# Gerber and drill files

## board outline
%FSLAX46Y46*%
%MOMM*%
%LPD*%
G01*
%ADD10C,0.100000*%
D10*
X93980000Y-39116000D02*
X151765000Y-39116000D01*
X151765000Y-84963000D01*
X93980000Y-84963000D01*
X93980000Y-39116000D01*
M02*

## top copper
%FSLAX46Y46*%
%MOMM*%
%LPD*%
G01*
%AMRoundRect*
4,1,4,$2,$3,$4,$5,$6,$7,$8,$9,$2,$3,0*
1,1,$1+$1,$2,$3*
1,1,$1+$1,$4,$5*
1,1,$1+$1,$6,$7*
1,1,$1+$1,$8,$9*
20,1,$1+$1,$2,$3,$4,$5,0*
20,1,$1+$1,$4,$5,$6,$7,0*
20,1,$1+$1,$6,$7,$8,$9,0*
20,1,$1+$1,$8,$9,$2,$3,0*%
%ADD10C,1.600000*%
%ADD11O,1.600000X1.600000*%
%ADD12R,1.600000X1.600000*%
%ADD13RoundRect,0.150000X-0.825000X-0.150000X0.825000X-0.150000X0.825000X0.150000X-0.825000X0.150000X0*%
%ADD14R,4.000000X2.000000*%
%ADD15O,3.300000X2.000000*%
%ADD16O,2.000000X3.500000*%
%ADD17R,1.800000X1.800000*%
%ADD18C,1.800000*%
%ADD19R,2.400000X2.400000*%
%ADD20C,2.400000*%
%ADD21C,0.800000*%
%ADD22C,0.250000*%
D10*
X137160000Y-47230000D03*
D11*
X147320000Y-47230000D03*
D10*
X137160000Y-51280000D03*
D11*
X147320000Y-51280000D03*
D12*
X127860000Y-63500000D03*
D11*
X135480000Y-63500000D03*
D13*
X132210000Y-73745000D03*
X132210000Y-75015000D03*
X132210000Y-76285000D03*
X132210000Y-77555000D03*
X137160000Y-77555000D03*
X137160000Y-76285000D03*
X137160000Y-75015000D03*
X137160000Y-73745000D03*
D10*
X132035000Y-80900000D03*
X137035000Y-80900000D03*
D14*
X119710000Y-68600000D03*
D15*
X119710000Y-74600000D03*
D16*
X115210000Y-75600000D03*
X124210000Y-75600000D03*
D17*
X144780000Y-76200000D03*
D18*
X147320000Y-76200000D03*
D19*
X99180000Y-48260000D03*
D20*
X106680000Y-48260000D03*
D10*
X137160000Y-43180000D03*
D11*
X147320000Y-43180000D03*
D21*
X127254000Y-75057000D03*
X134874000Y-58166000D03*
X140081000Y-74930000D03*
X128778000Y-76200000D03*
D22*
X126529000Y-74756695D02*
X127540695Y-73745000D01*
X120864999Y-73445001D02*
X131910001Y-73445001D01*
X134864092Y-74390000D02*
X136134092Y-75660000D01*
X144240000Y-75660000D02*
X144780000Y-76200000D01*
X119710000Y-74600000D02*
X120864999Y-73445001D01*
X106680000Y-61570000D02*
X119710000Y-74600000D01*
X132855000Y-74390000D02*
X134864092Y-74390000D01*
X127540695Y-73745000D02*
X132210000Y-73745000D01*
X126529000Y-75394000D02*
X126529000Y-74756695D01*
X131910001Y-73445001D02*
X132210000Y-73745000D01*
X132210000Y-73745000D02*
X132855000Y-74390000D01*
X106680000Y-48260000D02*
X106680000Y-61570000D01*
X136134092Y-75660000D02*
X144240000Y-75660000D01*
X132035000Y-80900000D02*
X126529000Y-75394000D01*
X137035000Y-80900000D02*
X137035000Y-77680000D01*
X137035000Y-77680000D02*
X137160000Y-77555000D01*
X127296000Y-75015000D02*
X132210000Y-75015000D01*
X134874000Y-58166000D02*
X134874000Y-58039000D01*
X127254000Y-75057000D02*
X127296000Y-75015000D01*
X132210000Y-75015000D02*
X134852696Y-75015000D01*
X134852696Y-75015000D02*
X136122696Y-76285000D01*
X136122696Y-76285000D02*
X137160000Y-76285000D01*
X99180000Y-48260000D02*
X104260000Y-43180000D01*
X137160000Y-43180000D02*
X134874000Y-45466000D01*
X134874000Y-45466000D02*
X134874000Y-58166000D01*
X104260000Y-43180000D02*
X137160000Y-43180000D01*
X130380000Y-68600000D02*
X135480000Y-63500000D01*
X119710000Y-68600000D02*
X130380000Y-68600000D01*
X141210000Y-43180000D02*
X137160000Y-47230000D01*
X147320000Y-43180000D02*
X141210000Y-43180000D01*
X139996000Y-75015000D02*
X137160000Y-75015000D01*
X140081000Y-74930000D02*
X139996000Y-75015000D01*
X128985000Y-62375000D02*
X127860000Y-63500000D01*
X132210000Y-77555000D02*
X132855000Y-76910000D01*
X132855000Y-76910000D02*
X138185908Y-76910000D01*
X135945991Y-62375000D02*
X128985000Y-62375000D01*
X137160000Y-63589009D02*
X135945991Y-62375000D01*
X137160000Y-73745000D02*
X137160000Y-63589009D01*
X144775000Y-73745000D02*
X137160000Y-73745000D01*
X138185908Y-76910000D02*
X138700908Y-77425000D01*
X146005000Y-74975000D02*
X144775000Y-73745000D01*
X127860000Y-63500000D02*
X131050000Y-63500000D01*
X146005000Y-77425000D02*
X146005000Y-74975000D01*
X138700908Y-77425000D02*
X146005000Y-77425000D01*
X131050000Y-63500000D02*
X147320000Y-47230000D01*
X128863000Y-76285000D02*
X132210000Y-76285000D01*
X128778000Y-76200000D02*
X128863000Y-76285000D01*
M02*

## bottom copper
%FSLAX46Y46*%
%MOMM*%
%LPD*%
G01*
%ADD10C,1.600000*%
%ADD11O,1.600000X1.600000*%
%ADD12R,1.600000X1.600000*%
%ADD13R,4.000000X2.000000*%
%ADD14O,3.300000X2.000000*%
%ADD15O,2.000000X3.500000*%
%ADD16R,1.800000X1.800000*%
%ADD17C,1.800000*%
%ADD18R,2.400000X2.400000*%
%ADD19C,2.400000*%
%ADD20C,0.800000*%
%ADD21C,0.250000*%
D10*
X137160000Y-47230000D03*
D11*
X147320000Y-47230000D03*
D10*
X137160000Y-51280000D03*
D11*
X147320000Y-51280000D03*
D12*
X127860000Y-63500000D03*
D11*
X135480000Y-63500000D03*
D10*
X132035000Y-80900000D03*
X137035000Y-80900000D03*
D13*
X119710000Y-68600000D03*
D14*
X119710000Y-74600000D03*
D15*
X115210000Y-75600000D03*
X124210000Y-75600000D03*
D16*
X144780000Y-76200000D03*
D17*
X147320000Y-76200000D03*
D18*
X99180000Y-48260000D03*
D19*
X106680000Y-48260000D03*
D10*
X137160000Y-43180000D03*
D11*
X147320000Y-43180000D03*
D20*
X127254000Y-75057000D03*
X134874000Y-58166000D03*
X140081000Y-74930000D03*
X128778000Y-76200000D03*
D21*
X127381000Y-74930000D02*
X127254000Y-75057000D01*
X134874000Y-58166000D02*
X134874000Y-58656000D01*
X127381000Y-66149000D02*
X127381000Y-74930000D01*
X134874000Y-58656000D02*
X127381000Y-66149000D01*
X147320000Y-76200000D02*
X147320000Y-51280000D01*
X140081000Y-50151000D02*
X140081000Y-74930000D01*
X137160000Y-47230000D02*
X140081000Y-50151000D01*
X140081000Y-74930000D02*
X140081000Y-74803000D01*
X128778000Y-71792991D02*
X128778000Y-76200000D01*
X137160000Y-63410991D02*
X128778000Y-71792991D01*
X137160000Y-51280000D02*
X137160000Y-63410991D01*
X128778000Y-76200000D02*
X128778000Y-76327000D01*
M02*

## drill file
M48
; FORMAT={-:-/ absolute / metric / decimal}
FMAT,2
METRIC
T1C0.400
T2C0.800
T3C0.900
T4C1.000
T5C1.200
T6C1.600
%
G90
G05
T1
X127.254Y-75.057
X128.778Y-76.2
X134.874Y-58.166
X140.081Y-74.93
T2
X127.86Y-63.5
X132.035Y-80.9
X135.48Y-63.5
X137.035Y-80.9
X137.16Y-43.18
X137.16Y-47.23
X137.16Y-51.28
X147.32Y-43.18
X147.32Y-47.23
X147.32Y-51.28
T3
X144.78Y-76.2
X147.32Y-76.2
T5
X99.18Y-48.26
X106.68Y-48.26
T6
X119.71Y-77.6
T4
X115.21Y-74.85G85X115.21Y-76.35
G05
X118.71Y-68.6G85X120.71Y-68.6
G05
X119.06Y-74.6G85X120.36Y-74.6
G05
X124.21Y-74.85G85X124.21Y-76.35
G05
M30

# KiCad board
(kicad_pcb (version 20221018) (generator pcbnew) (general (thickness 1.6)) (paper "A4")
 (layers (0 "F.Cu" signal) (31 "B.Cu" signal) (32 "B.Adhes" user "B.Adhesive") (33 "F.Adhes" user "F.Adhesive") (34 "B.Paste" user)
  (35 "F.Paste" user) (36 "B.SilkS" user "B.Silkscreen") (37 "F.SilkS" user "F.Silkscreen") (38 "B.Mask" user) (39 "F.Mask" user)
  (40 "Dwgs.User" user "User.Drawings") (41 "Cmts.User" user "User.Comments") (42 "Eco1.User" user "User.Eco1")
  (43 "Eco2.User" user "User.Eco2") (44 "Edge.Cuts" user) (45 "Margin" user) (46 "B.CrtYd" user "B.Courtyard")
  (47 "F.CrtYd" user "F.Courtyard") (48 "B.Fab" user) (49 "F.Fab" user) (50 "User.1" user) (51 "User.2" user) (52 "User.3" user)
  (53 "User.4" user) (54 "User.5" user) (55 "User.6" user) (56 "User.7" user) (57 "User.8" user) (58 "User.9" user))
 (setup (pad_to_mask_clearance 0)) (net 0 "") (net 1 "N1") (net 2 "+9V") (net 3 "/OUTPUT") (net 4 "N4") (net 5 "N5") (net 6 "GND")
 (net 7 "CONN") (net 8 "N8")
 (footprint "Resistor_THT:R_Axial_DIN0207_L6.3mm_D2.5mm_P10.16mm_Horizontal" (layer "F.Cu") (at 137.16 47.23)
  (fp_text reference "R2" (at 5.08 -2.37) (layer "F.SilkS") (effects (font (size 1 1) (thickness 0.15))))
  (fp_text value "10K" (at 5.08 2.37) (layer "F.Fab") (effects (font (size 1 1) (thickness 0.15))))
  (pad "1" thru_hole circle (at 0 0) (size 1.6 1.6) (drill 0.8) (layers "*.Cu" "*.Mask") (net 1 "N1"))
  (pad "2" thru_hole oval (at 10.16 0) (size 1.6 1.6) (drill 0.8) (layers "*.Cu" "*.Mask") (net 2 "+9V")))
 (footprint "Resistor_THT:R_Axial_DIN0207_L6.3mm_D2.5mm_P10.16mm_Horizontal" (layer "F.Cu") (at 137.16 51.28)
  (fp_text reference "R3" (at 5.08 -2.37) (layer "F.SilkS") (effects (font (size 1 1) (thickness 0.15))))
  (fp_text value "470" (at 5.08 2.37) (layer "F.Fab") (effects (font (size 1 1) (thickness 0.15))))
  (pad "1" thru_hole circle (at 0 0) (size 1.6 1.6) (drill 0.8) (layers "*.Cu" "*.Mask") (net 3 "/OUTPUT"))
  (pad "2" thru_hole oval (at 10.16 0) (size 1.6 1.6) (drill 0.8) (layers "*.Cu" "*.Mask") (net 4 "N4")))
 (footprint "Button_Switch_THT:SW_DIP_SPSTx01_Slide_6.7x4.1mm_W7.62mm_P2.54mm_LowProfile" (layer "F.Cu") (at 127.86 63.5)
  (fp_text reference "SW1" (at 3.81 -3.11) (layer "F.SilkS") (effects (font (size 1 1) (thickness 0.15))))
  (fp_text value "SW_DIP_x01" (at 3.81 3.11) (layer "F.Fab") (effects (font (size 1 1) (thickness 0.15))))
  (pad "1" thru_hole rect (at 0 0) (size 1.6 1.6) (drill 0.8) (layers "*.Cu" "*.Mask") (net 2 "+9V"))
  (pad "2" thru_hole oval (at 7.62 0) (size 1.6 1.6) (drill 0.8) (layers "*.Cu" "*.Mask") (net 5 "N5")))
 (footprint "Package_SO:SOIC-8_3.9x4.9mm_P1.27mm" (layer "F.Cu") (at 134.685 75.65)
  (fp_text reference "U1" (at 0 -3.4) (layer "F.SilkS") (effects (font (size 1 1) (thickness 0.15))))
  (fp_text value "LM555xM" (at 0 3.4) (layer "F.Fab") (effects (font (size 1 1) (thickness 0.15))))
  (pad "1" smd roundrect (at -2.475 -1.905) (size 1.95 0.6) (layers "F.Cu" "F.Paste" "F.Mask") (roundrect_rratio 0.25) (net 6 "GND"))
  (pad "2" smd roundrect (at -2.475 -0.635) (size 1.95 0.6) (layers "F.Cu" "F.Paste" "F.Mask") (roundrect_rratio 0.25) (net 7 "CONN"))
  (pad "3" smd roundrect (at -2.475 0.635) (size 1.95 0.6) (layers "F.Cu" "F.Paste" "F.Mask") (roundrect_rratio 0.25) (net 3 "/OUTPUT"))
  (pad "4" smd roundrect (at -2.475 1.905) (size 1.95 0.6) (layers "F.Cu" "F.Paste" "F.Mask") (roundrect_rratio 0.25) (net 2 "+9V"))
  (pad "5" smd roundrect (at 2.475 1.905) (size 1.95 0.6) (layers "F.Cu" "F.Paste" "F.Mask") (roundrect_rratio 0.25) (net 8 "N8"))
  (pad "6" smd roundrect (at 2.475 0.635) (size 1.95 0.6) (layers "F.Cu" "F.Paste" "F.Mask") (roundrect_rratio 0.25) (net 7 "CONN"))
  (pad "7" smd roundrect (at 2.475 -0.635) (size 1.95 0.6) (layers "F.Cu" "F.Paste" "F.Mask") (roundrect_rratio 0.25) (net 1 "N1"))
  (pad "8" smd roundrect (at 2.475 -1.905) (size 1.95 0.6) (layers "F.Cu" "F.Paste" "F.Mask") (roundrect_rratio 0.25) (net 2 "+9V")))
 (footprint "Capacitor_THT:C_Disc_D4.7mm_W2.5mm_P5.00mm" (layer "F.Cu") (at 132.035 80.9)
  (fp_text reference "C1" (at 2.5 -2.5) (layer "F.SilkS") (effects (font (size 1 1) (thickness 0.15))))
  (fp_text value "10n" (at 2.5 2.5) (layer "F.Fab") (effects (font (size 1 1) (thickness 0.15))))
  (pad "1" thru_hole circle (at 0 0) (size 1.6 1.6) (drill 0.8) (layers "*.Cu" "*.Mask") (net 6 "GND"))
  (pad "2" thru_hole circle (at 5 0) (size 1.6 1.6) (drill 0.8) (layers "*.Cu" "*.Mask") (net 8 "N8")))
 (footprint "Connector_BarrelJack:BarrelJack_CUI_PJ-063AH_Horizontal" (layer "F.Cu") (at 119.71 68.6)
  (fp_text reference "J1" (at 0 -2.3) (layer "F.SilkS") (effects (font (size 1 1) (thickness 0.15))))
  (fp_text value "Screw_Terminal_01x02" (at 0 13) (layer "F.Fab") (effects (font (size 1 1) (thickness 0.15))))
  (pad "" np_thru_hole circle (at 0 9) (size 1.6 1.6) (drill 1.6) (layers "*.Cu" "*.Mask"))
  (pad "1" thru_hole rect (at 0 0) (size 4 2) (drill oval 3 1) (layers "*.Cu" "*.Mask") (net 5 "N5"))
  (pad "2" thru_hole oval (at 0 6) (size 3.3 2) (drill oval 2.3 1) (layers "*.Cu" "*.Mask") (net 6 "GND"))
  (pad "MP" thru_hole oval (at -4.5 7) (size 2 3.5) (drill oval 1 2.5) (layers "*.Cu" "*.Mask"))
  (pad "MP" thru_hole oval (at 4.5 7) (size 2 3.5) (drill oval 1 2.5) (layers "*.Cu" "*.Mask")))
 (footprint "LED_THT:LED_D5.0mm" (layer "F.Cu") (at 144.78 76.2)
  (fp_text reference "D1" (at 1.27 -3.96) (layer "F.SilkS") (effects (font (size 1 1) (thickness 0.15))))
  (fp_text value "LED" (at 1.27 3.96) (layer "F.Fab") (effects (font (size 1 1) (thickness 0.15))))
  (pad "1" thru_hole rect (at 0 0) (size 1.8 1.8) (drill 0.9) (layers "*.Cu" "*.Mask") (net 6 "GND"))
  (pad "2" thru_hole circle (at 2.54 0) (size 1.8 1.8) (drill 0.9) (layers "*.Cu" "*.Mask") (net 4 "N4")))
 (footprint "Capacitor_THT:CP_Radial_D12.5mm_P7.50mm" (layer "F.Cu") (at 99.18 48.26)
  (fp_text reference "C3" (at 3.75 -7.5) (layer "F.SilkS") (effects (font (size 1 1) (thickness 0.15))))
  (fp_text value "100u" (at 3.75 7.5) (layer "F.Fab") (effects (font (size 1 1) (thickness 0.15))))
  (pad "1" thru_hole rect (at 0 0) (size 2.4 2.4) (drill 1.2) (layers "*.Cu" "*.Mask") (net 7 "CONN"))
  (pad "2" thru_hole circle (at 7.5 0) (size 2.4 2.4) (drill 1.2) (layers "*.Cu" "*.Mask") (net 6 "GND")))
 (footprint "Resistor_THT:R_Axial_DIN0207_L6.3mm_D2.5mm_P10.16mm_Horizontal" (layer "F.Cu") (at 137.16 43.18)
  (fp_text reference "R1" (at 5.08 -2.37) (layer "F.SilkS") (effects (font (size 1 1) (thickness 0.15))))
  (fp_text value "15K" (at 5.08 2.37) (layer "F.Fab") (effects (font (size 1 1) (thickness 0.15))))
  (pad "1" thru_hole circle (at 0 0) (size 1.6 1.6) (drill 0.8) (layers "*.Cu" "*.Mask") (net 7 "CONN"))
  (pad "2" thru_hole oval (at 10.16 0) (size 1.6 1.6) (drill 0.8) (layers "*.Cu" "*.Mask") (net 1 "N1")))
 (gr_rect (start 93.98 39.116) (end 151.765 84.963) (stroke (width 0.1) (type default)) (fill none) (layer "Edge.Cuts"))
 (segment (start 126.529 74.756695) (end 127.540695 73.745) (width 0.25) (layer "F.Cu") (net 6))
 (segment (start 120.864999 73.445001) (end 131.910001 73.445001) (width 0.25) (layer "F.Cu") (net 6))
 (segment (start 134.864092 74.39) (end 136.134092 75.66) (width 0.25) (layer "F.Cu") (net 6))
 (segment (start 144.24 75.66) (end 144.78 76.2) (width 0.25) (layer "F.Cu") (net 6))
 (segment (start 119.71 74.6) (end 120.864999 73.445001) (width 0.25) (layer "F.Cu") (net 6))
 (segment (start 106.68 61.57) (end 119.71 74.6) (width 0.25) (layer "F.Cu") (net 6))
 (segment (start 132.855 74.39) (end 134.864092 74.39) (width 0.25) (layer "F.Cu") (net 6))
 (segment (start 127.540695 73.745) (end 132.21 73.745) (width 0.25) (layer "F.Cu") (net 6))
 (segment (start 126.529 75.394) (end 126.529 74.756695) (width 0.25) (layer "F.Cu") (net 6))
 (segment (start 131.910001 73.445001) (end 132.21 73.745) (width 0.25) (layer "F.Cu") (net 6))
 (segment (start 132.21 73.745) (end 132.855 74.39) (width 0.25) (layer "F.Cu") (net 6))
 (segment (start 106.68 48.26) (end 106.68 61.57) (width 0.25) (layer "F.Cu") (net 6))
 (segment (start 136.134092 75.66) (end 144.24 75.66) (width 0.25) (layer "F.Cu") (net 6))
 (segment (start 132.035 80.9) (end 126.529 75.394) (width 0.25) (layer "F.Cu") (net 6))
 (segment (start 137.035 80.9) (end 137.035 77.68) (width 0.25) (layer "F.Cu") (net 8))
 (segment (start 137.035 77.68) (end 137.16 77.555) (width 0.25) (layer "F.Cu") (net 8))
 (segment (start 127.296 75.015) (end 132.21 75.015) (width 0.25) (layer "F.Cu") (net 7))
 (segment (start 134.874 58.166) (end 134.874 58.039) (width 0.25) (layer "F.Cu") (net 7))
 (segment (start 127.254 75.057) (end 127.296 75.015) (width 0.25) (layer "F.Cu") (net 7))
 (segment (start 132.21 75.015) (end 134.852696 75.015) (width 0.25) (layer "F.Cu") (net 7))
 (segment (start 134.852696 75.015) (end 136.122696 76.285) (width 0.25) (layer "F.Cu") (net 7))
 (segment (start 136.122696 76.285) (end 137.16 76.285) (width 0.25) (layer "F.Cu") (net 7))
 (segment (start 99.18 48.26) (end 104.26 43.18) (width 0.25) (layer "F.Cu") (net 7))
 (segment (start 137.16 43.18) (end 134.874 45.466) (width 0.25) (layer "F.Cu") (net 7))
 (segment (start 134.874 45.466) (end 134.874 58.166) (width 0.25) (layer "F.Cu") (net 7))
 (segment (start 104.26 43.18) (end 137.16 43.18) (width 0.25) (layer "F.Cu") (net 7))
 (via (at 127.254 75.057) (size 0.8) (drill 0.4) (layers "F.Cu" "B.Cu") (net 7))
 (via (at 134.874 58.166) (size 0.8) (drill 0.4) (layers "F.Cu" "B.Cu") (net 7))
 (segment (start 127.381 74.93) (end 127.254 75.057) (width 0.25) (layer "B.Cu") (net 7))
 (segment (start 134.874 58.166) (end 134.874 58.656) (width 0.25) (layer "B.Cu") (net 7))
 (segment (start 127.381 66.149) (end 127.381 74.93) (width 0.25) (layer "B.Cu") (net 7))
 (segment (start 134.874 58.656) (end 127.381 66.149) (width 0.25) (layer "B.Cu") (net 7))
 (segment (start 147.32 76.2) (end 147.32 51.28) (width 0.25) (layer "B.Cu") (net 4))
 (segment (start 130.38 68.6) (end 135.48 63.5) (width 0.25) (layer "F.Cu") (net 5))
 (segment (start 119.71 68.6) (end 130.38 68.6) (width 0.25) (layer "F.Cu") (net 5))
 (segment (start 141.21 43.18) (end 137.16 47.23) (width 0.25) (layer "F.Cu") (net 1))
 (segment (start 147.32 43.18) (end 141.21 43.18) (width 0.25) (layer "F.Cu") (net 1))
 (segment (start 139.996 75.015) (end 137.16 75.015) (width 0.25) (layer "F.Cu") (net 1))
 (segment (start 140.081 74.93) (end 139.996 75.015) (width 0.25) (layer "F.Cu") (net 1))
 (via (at 140.081 74.93) (size 0.8) (drill 0.4) (layers "F.Cu" "B.Cu") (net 1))
 (segment (start 140.081 50.151) (end 140.081 74.93) (width 0.25) (layer "B.Cu") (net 1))
 (segment (start 137.16 47.23) (end 140.081 50.151) (width 0.25) (layer "B.Cu") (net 1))
 (segment (start 140.081 74.93) (end 140.081 74.803) (width 0.25) (layer "B.Cu") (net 1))
 (segment (start 128.985 62.375) (end 127.86 63.5) (width 0.25) (layer "F.Cu") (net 2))
 (segment (start 132.21 77.555) (end 132.855 76.91) (width 0.25) (layer "F.Cu") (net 2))
 (segment (start 132.855 76.91) (end 138.185908 76.91) (width 0.25) (layer "F.Cu") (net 2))
 (segment (start 135.945991 62.375) (end 128.985 62.375) (width 0.25) (layer "F.Cu") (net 2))
 (segment (start 137.16 63.589009) (end 135.945991 62.375) (width 0.25) (layer "F.Cu") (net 2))
 (segment (start 137.16 73.745) (end 137.16 63.589009) (width 0.25) (layer "F.Cu") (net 2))
 (segment (start 144.775 73.745) (end 137.16 73.745) (width 0.25) (layer "F.Cu") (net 2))
 (segment (start 138.185908 76.91) (end 138.700908 77.425) (width 0.25) (layer "F.Cu") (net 2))
 (segment (start 146.005 74.975) (end 144.775 73.745) (width 0.25) (layer "F.Cu") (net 2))
 (segment (start 127.86 63.5) (end 131.05 63.5) (width 0.25) (layer "F.Cu") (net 2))
 (segment (start 146.005 77.425) (end 146.005 74.975) (width 0.25) (layer "F.Cu") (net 2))
 (segment (start 138.700908 77.425) (end 146.005 77.425) (width 0.25) (layer "F.Cu") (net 2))
 (segment (start 131.05 63.5) (end 147.32 47.23) (width 0.25) (layer "F.Cu") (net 2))
 (segment (start 128.863 76.285) (end 132.21 76.285) (width 0.25) (layer "F.Cu") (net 3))
 (segment (start 128.778 76.2) (end 128.863 76.285) (width 0.25) (layer "F.Cu") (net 3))
 (via (at 128.778 76.2) (size 0.8) (drill 0.4) (layers "F.Cu" "B.Cu") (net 3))
 (segment (start 128.778 71.792991) (end 128.778 76.2) (width 0.25) (layer "B.Cu") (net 3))
 (segment (start 137.16 63.410991) (end 128.778 71.792991) (width 0.25) (layer "B.Cu") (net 3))
 (segment (start 137.16 51.28) (end 137.16 63.410991) (width 0.25) (layer "B.Cu") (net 3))
 (segment (start 128.778 76.2) (end 128.778 76.327) (width 0.25) (layer "B.Cu") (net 3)))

